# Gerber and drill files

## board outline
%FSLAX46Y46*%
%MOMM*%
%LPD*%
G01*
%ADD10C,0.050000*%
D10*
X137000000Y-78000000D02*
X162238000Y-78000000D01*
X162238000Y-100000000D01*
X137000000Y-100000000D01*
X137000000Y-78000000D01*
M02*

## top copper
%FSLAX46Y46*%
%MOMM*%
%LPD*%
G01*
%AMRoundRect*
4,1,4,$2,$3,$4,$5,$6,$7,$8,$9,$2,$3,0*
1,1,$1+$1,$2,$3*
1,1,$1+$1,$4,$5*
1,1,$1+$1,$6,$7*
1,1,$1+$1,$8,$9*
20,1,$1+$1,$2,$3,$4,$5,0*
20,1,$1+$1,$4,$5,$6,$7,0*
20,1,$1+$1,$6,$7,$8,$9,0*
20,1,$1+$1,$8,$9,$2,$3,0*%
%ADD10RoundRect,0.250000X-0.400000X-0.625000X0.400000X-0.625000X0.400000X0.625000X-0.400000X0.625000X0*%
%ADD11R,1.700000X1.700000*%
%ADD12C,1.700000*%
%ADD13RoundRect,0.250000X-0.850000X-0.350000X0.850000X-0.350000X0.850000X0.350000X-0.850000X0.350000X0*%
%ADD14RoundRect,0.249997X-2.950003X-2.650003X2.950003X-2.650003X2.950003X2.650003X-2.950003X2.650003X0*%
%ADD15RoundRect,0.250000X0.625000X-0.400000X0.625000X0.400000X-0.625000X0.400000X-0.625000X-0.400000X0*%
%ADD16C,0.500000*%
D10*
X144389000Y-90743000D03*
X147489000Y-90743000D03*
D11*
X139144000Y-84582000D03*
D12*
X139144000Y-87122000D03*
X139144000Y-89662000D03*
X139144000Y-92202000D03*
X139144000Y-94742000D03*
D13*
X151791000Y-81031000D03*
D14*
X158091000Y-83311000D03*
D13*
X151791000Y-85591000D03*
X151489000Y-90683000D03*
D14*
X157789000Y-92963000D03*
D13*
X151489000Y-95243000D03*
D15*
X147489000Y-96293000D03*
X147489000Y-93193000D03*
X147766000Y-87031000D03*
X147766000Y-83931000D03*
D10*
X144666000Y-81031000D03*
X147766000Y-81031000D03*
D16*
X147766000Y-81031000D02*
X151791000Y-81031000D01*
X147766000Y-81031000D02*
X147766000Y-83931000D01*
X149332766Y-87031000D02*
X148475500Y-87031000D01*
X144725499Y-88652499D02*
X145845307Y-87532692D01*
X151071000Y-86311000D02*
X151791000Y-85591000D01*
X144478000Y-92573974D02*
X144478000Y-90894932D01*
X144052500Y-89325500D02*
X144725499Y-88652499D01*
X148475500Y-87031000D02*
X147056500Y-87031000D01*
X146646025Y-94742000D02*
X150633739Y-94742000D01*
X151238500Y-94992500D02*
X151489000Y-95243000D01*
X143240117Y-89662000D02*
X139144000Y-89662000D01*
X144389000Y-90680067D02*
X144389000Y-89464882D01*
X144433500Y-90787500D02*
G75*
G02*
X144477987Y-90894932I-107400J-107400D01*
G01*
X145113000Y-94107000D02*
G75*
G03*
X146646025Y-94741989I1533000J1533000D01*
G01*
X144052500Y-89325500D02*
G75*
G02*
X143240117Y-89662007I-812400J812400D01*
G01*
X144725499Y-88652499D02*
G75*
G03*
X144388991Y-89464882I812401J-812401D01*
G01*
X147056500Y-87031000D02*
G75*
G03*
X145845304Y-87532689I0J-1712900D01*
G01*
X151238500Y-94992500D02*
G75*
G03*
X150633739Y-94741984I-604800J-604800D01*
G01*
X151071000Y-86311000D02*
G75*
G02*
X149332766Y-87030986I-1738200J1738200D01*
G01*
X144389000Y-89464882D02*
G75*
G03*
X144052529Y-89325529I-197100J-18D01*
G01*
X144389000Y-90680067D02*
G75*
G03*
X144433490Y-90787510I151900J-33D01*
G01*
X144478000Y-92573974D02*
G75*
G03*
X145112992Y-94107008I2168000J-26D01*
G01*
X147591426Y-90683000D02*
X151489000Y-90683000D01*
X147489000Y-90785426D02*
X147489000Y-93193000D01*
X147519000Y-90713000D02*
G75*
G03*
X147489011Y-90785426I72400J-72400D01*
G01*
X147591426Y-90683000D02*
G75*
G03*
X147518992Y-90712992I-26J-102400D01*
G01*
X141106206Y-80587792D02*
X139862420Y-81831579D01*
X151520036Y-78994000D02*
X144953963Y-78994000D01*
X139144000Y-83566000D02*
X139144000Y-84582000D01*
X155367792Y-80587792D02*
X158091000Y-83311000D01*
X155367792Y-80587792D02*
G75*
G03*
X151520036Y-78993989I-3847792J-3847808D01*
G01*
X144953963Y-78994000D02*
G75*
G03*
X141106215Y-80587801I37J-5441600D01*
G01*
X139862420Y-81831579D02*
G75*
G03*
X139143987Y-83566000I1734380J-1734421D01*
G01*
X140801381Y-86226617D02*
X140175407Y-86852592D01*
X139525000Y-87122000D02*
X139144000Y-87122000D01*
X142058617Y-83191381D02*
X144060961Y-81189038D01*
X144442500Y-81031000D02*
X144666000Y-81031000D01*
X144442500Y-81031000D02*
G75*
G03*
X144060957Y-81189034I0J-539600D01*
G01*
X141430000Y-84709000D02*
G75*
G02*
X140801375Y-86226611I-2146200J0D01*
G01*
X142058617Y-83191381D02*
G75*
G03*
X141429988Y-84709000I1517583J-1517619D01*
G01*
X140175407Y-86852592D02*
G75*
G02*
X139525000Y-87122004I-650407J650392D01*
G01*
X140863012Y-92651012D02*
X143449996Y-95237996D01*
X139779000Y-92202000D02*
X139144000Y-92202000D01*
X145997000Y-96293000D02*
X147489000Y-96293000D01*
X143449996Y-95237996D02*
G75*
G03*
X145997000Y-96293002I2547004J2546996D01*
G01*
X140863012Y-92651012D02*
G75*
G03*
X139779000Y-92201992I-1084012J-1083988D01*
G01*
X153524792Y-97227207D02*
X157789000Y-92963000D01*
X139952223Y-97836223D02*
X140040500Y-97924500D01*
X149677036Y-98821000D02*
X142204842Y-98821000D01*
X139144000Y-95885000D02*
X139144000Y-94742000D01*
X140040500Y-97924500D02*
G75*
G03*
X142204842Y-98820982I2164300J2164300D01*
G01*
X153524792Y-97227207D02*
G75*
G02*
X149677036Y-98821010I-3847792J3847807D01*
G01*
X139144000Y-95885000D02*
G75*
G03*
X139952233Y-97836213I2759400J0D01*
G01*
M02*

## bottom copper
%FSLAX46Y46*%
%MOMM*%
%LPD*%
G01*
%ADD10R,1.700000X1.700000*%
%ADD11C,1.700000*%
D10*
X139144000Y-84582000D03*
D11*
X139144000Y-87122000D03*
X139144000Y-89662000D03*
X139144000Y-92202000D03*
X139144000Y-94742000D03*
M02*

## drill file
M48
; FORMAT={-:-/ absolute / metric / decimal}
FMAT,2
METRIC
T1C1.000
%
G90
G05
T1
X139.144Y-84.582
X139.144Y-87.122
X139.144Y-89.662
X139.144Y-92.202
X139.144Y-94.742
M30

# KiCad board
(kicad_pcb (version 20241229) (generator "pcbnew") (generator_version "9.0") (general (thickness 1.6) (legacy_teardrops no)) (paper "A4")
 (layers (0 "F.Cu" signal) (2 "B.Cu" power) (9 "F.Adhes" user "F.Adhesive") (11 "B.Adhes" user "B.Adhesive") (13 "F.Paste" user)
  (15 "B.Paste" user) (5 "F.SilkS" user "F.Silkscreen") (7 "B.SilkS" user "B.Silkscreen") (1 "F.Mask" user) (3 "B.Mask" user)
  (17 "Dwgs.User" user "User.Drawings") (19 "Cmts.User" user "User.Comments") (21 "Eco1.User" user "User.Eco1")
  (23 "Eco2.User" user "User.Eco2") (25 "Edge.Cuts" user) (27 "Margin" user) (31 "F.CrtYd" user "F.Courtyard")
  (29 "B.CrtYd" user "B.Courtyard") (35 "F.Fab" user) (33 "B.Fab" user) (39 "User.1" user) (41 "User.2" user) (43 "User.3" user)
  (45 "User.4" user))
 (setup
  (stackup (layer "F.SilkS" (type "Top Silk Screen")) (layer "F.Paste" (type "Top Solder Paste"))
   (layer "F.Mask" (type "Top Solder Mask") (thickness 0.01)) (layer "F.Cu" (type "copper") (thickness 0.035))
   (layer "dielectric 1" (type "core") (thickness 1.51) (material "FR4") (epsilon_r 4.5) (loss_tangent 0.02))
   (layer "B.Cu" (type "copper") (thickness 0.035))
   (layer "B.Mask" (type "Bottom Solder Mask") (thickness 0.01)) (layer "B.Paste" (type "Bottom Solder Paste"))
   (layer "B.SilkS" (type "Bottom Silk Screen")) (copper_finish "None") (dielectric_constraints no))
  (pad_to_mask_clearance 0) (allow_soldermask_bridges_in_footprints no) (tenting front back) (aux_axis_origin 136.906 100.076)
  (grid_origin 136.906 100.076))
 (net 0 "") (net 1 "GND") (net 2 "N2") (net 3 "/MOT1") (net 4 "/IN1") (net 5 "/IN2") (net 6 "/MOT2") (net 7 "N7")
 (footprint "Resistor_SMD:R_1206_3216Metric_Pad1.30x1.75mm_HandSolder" (layer "F.Cu") (at 145.939 90.743)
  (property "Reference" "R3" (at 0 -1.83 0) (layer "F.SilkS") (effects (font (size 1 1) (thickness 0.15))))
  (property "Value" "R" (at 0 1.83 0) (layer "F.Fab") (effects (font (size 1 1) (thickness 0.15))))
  (pad "1" smd roundrect (at -1.55 0) (size 1.3 1.75) (layers "F.Cu" "F.Mask" "F.Paste") (roundrect_rratio 0.192308) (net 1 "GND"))
  (pad "2" smd roundrect (at 1.55 0) (size 1.3 1.75) (layers "F.Cu" "F.Mask" "F.Paste") (roundrect_rratio 0.192308) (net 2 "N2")))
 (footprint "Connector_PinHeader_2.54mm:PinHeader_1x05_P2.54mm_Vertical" (layer "F.Cu") (at 139.144 84.582)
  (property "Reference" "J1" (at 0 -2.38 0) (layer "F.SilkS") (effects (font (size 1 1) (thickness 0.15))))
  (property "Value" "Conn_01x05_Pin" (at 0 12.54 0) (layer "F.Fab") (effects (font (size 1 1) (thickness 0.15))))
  (pad "1" thru_hole rect (at 0 0) (size 1.7 1.7) (drill 1) (layers "*.Cu" "*.Mask") (remove_unused_layers no) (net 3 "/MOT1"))
  (pad "2" thru_hole circle (at 0 2.54) (size 1.7 1.7) (drill 1) (layers "*.Cu" "*.Mask") (remove_unused_layers no) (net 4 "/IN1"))
  (pad "3" thru_hole circle (at 0 5.08) (size 1.7 1.7) (drill 1) (layers "*.Cu" "*.Mask") (remove_unused_layers no) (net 1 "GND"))
  (pad "4" thru_hole circle (at 0 7.62) (size 1.7 1.7) (drill 1) (layers "*.Cu" "*.Mask") (remove_unused_layers no) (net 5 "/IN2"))
  (pad "5" thru_hole circle (at 0 10.16) (size 1.7 1.7) (drill 1) (layers "*.Cu" "*.Mask") (remove_unused_layers no) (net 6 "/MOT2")))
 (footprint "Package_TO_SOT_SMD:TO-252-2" (layer "F.Cu") (at 156.831 83.311)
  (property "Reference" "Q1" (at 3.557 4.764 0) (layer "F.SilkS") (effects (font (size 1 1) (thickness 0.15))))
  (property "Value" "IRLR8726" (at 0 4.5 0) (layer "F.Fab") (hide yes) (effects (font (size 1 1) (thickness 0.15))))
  (pad "" smd roundrect (at -0.415 -1.525) (size 3.05 2.75) (layers "F.Paste") (roundrect_rratio 0.090909))
  (pad "" smd roundrect (at -0.415 1.525) (size 3.05 2.75) (layers "F.Paste") (roundrect_rratio 0.090909))
  (pad "" smd roundrect (at 2.935 -1.525) (size 3.05 2.75) (layers "F.Paste") (roundrect_rratio 0.090909))
  (pad "" smd roundrect (at 2.935 1.525) (size 3.05 2.75) (layers "F.Paste") (roundrect_rratio 0.090909))
  (pad "1" smd roundrect (at -5.04 -2.28) (size 2.2 1.2) (layers "F.Cu" "F.Mask" "F.Paste") (roundrect_rratio 0.208333) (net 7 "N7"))
  (pad "2" smd roundrect (at 1.26 0) (size 6.4 5.8) (layers "F.Cu" "F.Mask") (roundrect_rratio 0.043103) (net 3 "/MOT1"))
  (pad "3" smd roundrect (at -5.04 2.28) (size 2.2 1.2) (layers "F.Cu" "F.Mask" "F.Paste") (roundrect_rratio 0.208333) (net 1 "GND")))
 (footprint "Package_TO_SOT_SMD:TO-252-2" (layer "F.Cu") (at 156.529 92.963)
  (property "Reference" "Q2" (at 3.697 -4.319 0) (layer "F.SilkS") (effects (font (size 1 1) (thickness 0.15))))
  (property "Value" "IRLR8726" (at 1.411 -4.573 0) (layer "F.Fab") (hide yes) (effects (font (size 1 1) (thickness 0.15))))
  (pad "" smd roundrect (at -0.415 -1.525) (size 3.05 2.75) (layers "F.Paste") (roundrect_rratio 0.090909))
  (pad "" smd roundrect (at -0.415 1.525) (size 3.05 2.75) (layers "F.Paste") (roundrect_rratio 0.090909))
  (pad "" smd roundrect (at 2.935 -1.525) (size 3.05 2.75) (layers "F.Paste") (roundrect_rratio 0.090909))
  (pad "" smd roundrect (at 2.935 1.525) (size 3.05 2.75) (layers "F.Paste") (roundrect_rratio 0.090909))
  (pad "1" smd roundrect (at -5.04 -2.28) (size 2.2 1.2) (layers "F.Cu" "F.Mask" "F.Paste") (roundrect_rratio 0.208333) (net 2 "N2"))
  (pad "2" smd roundrect (at 1.26 0) (size 6.4 5.8) (layers "F.Cu" "F.Mask") (roundrect_rratio 0.043103) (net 6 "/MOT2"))
  (pad "3" smd roundrect (at -5.04 2.28) (size 2.2 1.2) (layers "F.Cu" "F.Mask" "F.Paste") (roundrect_rratio 0.208333) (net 1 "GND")))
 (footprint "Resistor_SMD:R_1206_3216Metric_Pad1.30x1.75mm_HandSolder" (layer "F.Cu") (at 147.489 94.743 90)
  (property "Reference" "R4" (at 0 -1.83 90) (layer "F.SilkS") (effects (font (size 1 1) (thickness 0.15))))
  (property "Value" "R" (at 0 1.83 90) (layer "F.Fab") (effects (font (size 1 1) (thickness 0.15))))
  (pad "1" smd roundrect (at -1.55 0 90) (size 1.3 1.75) (layers "F.Cu" "F.Mask" "F.Paste") (roundrect_rratio 0.192308) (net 5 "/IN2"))
  (pad "2" smd roundrect (at 1.55 0 90) (size 1.3 1.75) (layers "F.Cu" "F.Mask" "F.Paste") (roundrect_rratio 0.192308) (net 2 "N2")))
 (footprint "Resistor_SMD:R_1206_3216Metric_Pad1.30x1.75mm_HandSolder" (layer "F.Cu") (at 147.766 85.481 90)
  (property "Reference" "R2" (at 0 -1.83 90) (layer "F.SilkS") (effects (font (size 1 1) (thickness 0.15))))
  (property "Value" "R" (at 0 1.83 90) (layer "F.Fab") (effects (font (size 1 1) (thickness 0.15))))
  (pad "1" smd roundrect (at -1.55 0 90) (size 1.3 1.75) (layers "F.Cu" "F.Mask" "F.Paste") (roundrect_rratio 0.192308) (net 1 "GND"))
  (pad "2" smd roundrect (at 1.55 0 90) (size 1.3 1.75) (layers "F.Cu" "F.Mask" "F.Paste") (roundrect_rratio 0.192308) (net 7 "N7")))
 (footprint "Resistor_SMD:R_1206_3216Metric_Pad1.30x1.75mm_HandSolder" (layer "F.Cu") (at 146.216 81.031)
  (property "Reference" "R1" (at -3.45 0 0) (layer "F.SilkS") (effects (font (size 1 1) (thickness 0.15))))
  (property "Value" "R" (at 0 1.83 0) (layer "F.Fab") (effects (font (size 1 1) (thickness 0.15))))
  (pad "1" smd roundrect (at -1.55 0) (size 1.3 1.75) (layers "F.Cu" "F.Mask" "F.Paste") (roundrect_rratio 0.192308) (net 4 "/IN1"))
  (pad "2" smd roundrect (at 1.55 0) (size 1.3 1.75) (layers "F.Cu" "F.Mask" "F.Paste") (roundrect_rratio 0.192308) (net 7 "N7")))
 (gr_rect (start 137 78) (end 162.238 100) (stroke (width 0.05) (type default)) (fill no) (layer "Edge.Cuts"))
 (segment (start 147.766 81.031) (end 151.791 81.031) (width 0.5) (layer "F.Cu") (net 7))
 (segment (start 147.766 81.031) (end 147.766 83.931) (width 0.5) (layer "F.Cu") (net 7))
 (segment (start 149.332766 87.031) (end 148.4755 87.031) (width 0.5) (layer "F.Cu") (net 1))
 (segment (start 144.725499 88.652499) (end 145.845307 87.532692) (width 0.5) (layer "F.Cu") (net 1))
 (segment (start 151.071 86.311) (end 151.791 85.591) (width 0.5) (layer "F.Cu") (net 1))
 (segment (start 144.478 92.573974) (end 144.478 90.894932) (width 0.5) (layer "F.Cu") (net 1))
 (segment (start 144.0525 89.3255) (end 144.725499 88.652499) (width 0.5) (layer "F.Cu") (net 1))
 (segment (start 148.4755 87.031) (end 147.0565 87.031) (width 0.5) (layer "F.Cu") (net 1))
 (segment (start 146.646025 94.742) (end 150.633739 94.742) (width 0.5) (layer "F.Cu") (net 1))
 (segment (start 151.2385 94.9925) (end 151.489 95.243) (width 0.5) (layer "F.Cu") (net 1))
 (segment (start 143.240117 89.662) (end 139.144 89.662) (width 0.5) (layer "F.Cu") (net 1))
 (segment (start 144.389 90.680067) (end 144.389 89.464882) (width 0.5) (layer "F.Cu") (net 1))
 (arc (start 144.4335 90.7875) (mid 144.466434 90.83679) (end 144.478 90.894932) (width 0.5) (layer "F.Cu") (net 1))
 (arc (start 145.113 94.107) (mid 145.816357 94.576968) (end 146.646025 94.742) (width 0.5) (layer "F.Cu") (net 1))
 (arc (start 144.0525 89.3255) (mid 143.679775 89.574546) (end 143.240117 89.662) (width 0.5) (layer "F.Cu") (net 1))
 (arc (start 144.725499 88.652499) (mid 144.476453 89.025223) (end 144.389 89.464882) (width 0.5) (layer "F.Cu") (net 1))
 (arc (start 147.0565 87.031) (mid 146.401007 87.161385) (end 145.845307 87.532692) (width 0.5) (layer "F.Cu") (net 1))
 (arc (start 151.2385 94.9925) (mid 150.961033 94.807102) (end 150.633739 94.742) (width 0.5) (layer "F.Cu") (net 1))
 (arc (start 151.071 86.311) (mid 150.273491 86.843878) (end 149.332766 87.031) (width 0.5) (layer "F.Cu") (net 1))
 (arc (start 144.389 89.464882) (mid 144.267316 89.28277) (end 144.0525 89.3255) (width 0.5) (layer "F.Cu") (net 1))
 (arc (start 144.389 90.680067) (mid 144.400565 90.738209) (end 144.4335 90.7875) (width 0.5) (layer "F.Cu") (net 1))
 (arc (start 144.478 92.573974) (mid 144.643031 93.403641) (end 145.113 94.107) (width 0.5) (layer "F.Cu") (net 1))
 (segment (start 147.591426 90.683) (end 151.489 90.683) (width 0.5) (layer "F.Cu") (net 2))
 (segment (start 147.489 90.785426) (end 147.489 93.193) (width 0.5) (layer "F.Cu") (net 2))
 (arc (start 147.519 90.713) (mid 147.496796 90.746229) (end 147.489 90.785426) (width 0.5) (layer "F.Cu") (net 2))
 (arc (start 147.591426 90.683) (mid 147.552229 90.690796) (end 147.519 90.713) (width 0.5) (layer "F.Cu") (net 2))
 (segment (start 141.106206 80.587792) (end 139.86242 81.831579) (width 0.5) (layer "F.Cu") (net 3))
 (segment (start 151.520036 78.994) (end 144.953963 78.994) (width 0.5) (layer "F.Cu") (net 3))
 (segment (start 139.144 83.566) (end 139.144 84.582) (width 0.5) (layer "F.Cu") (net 3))
 (segment (start 155.367792 80.587792) (end 158.091 83.311) (width 0.5) (layer "F.Cu") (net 3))
 (arc (start 155.367792 80.587792) (mid 153.602426 79.408213) (end 151.520036 78.994) (width 0.5) (layer "F.Cu") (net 3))
 (arc (start 144.953963 78.994) (mid 142.871572 79.408213) (end 141.106206 80.587792) (width 0.5) (layer "F.Cu") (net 3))
 (arc (start 139.86242 81.831579) (mid 139.330711 82.627338) (end 139.144 83.566) (width 0.5) (layer "F.Cu") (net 3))
 (segment (start 140.801381 86.226617) (end 140.175407 86.852592) (width 0.5) (layer "F.Cu") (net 4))
 (segment (start 139.525 87.122) (end 139.144 87.122) (width 0.5) (layer "F.Cu") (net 4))
 (segment (start 142.058617 83.191381) (end 144.060961 81.189038) (width 0.5) (layer "F.Cu") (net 4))
 (segment (start 144.4425 81.031) (end 144.666 81.031) (width 0.5) (layer "F.Cu") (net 4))
 (arc (start 144.4425 81.031) (mid 144.236012 81.072072) (end 144.060961 81.189038) (width 0.5) (layer "F.Cu") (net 4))
 (arc (start 141.43 84.709) (mid 141.266627 85.530328) (end 140.801381 86.226617) (width 0.5) (layer "F.Cu") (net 4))
 (arc (start 142.058617 83.191381) (mid 141.593372 83.88767) (end 141.43 84.709) (width 0.5) (layer "F.Cu") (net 4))
 (arc (start 140.175407 86.852592) (mid 139.876997 87.051983) (end 139.525 87.122) (width 0.5) (layer "F.Cu") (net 4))
 (segment (start 140.863012 92.651012) (end 143.449996 95.237996) (width 0.5) (layer "F.Cu") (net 5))
 (segment (start 139.779 92.202) (end 139.144 92.202) (width 0.5) (layer "F.Cu") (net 5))
 (segment (start 145.997 96.293) (end 147.489 96.293) (width 0.5) (layer "F.Cu") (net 5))
 (arc (start 143.449996 95.237996) (mid 144.618571 96.018813) (end 145.997 96.293) (width 0.5) (layer "F.Cu") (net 5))
 (arc (start 140.863012 92.651012) (mid 140.365663 92.318694) (end 139.779 92.202) (width 0.5) (layer "F.Cu") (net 5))
 (segment (start 153.524792 97.227207) (end 157.789 92.963) (width 0.5) (layer "F.Cu") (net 6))
 (segment (start 139.952223 97.836223) (end 140.0405 97.9245) (width 0.5) (layer "F.Cu") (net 6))
 (segment (start 149.677036 98.821) (end 142.204842 98.821) (width 0.5) (layer "F.Cu") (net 6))
 (segment (start 139.144 95.885) (end 139.144 94.742) (width 0.5) (layer "F.Cu") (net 6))
 (arc (start 140.0405 97.9245) (mid 141.033508 98.588007) (end 142.204842 98.821) (width 0.5) (layer "F.Cu") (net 6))
 (arc (start 153.524792 97.227207) (mid 151.759426 98.406786) (end 149.677036 98.821) (width 0.5) (layer "F.Cu") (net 6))
 (arc (start 139.144 95.885) (mid 139.35405 96.940994) (end 139.952223 97.836223) (width 0.5) (layer "F.Cu") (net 6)))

